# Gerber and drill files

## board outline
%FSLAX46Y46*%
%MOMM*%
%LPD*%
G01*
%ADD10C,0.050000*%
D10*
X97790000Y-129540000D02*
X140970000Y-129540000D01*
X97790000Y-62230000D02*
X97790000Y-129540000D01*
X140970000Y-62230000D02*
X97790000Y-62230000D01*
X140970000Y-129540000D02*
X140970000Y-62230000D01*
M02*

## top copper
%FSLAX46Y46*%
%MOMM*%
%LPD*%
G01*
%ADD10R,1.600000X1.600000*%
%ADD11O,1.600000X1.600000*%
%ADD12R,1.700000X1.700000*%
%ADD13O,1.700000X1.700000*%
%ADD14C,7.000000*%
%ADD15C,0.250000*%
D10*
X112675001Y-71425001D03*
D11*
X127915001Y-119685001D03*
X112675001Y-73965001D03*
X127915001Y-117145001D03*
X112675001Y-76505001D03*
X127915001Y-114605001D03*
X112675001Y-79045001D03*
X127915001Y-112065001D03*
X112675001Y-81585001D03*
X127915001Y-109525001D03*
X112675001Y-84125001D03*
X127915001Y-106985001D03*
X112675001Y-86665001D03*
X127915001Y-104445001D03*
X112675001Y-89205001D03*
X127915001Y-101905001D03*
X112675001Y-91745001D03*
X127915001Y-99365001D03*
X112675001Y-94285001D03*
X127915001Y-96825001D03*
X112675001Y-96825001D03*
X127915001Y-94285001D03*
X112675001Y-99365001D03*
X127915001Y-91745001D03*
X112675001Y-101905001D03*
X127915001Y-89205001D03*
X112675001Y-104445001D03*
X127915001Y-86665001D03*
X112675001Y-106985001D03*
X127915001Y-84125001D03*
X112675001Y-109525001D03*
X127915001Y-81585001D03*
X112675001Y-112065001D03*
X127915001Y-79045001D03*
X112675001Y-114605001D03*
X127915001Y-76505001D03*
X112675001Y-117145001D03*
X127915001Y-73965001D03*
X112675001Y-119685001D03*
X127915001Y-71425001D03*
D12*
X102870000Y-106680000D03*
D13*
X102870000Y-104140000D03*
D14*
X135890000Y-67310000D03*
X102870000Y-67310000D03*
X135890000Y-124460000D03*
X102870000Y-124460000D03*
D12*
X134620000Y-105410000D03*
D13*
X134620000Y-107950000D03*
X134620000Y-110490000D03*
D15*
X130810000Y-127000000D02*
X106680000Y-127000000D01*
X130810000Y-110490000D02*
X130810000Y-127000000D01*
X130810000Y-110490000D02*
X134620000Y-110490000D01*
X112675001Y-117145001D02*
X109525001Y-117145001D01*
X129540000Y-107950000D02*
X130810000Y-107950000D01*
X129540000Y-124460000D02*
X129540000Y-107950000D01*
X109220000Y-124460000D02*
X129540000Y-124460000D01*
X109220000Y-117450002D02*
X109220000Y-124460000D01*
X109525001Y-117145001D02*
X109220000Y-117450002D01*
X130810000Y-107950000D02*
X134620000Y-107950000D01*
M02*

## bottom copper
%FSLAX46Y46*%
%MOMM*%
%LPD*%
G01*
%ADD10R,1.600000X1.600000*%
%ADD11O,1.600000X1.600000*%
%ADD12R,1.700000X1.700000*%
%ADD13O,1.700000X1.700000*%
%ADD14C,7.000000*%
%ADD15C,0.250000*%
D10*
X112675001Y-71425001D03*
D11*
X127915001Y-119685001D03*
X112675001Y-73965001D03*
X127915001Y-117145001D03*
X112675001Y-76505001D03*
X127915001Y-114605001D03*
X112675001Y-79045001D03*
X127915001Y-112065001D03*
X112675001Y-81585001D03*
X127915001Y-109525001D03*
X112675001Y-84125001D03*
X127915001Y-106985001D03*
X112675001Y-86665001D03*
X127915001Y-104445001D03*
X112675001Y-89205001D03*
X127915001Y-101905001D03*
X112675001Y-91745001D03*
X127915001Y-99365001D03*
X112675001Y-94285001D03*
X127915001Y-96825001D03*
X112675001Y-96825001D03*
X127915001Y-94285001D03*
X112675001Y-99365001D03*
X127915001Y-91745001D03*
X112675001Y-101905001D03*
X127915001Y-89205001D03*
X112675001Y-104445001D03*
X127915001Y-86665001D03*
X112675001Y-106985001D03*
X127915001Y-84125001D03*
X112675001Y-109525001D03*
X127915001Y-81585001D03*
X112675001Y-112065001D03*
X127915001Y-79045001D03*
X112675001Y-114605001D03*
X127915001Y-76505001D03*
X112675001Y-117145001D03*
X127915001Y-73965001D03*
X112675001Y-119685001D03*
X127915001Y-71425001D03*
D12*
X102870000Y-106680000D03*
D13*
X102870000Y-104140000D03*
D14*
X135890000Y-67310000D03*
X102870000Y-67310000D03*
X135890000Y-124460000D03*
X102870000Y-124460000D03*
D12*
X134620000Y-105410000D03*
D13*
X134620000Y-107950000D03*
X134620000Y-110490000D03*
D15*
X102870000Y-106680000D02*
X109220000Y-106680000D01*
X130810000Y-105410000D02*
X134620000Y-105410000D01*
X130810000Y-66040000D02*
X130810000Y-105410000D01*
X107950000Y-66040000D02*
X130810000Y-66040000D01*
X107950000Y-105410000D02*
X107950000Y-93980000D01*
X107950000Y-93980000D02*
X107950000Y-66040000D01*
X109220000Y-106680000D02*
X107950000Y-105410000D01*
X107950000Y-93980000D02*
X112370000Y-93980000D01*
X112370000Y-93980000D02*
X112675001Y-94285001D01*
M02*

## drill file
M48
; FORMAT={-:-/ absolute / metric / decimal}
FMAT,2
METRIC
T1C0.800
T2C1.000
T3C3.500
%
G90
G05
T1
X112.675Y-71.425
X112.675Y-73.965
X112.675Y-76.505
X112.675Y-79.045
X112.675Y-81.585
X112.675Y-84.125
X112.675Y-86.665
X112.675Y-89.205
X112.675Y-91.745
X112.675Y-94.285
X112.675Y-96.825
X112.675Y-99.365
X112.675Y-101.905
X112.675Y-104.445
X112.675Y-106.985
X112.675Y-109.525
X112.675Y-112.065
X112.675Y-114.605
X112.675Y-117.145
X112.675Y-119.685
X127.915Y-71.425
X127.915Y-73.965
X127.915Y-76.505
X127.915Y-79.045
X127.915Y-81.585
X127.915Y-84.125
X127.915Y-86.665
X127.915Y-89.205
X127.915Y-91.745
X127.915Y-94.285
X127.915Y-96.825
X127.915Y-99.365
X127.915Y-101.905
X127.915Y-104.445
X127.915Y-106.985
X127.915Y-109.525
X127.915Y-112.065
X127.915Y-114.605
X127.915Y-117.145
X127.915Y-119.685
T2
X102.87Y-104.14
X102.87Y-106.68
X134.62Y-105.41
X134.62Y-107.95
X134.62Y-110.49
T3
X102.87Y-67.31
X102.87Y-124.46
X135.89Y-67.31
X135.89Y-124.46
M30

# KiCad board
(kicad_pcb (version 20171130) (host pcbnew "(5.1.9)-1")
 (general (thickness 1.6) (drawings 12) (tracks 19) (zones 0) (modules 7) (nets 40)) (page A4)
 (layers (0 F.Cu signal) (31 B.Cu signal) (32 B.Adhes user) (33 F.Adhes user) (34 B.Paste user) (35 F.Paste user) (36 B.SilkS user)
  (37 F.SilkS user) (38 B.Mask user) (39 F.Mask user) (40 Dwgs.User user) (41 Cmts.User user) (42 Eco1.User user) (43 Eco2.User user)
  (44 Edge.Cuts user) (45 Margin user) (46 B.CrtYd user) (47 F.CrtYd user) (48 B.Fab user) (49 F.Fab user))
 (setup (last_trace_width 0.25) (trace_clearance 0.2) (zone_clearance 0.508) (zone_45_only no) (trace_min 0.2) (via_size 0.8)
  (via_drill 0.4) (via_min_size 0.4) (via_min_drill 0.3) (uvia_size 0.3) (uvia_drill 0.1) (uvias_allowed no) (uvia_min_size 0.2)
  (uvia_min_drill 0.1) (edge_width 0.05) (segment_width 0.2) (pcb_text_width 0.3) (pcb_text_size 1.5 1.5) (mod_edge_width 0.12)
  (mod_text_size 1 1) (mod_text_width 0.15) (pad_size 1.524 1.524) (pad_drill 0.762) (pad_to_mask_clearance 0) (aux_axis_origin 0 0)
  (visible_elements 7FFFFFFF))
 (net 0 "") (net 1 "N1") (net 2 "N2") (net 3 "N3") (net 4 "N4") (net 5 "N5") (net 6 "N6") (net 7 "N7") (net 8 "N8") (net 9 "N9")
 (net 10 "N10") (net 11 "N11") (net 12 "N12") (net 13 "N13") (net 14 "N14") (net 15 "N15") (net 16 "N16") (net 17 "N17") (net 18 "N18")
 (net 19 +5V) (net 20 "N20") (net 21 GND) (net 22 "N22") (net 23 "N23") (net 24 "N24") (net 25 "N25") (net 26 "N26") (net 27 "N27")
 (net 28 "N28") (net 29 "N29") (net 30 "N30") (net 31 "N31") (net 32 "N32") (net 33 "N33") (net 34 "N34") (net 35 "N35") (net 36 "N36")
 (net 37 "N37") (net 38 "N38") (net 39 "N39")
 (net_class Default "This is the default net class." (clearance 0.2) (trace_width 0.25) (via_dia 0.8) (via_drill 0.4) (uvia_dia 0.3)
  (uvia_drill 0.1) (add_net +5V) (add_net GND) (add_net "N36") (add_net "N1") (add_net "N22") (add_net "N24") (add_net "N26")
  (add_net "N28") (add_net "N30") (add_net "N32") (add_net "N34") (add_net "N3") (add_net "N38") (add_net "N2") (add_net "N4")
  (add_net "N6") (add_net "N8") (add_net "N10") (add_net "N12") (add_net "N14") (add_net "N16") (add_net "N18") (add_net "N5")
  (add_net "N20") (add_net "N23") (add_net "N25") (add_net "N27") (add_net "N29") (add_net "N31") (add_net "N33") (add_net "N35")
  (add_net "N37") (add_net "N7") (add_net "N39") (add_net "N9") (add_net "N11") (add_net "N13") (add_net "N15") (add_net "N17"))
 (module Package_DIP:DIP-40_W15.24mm (layer F.Cu) (at 112.675001 71.425001)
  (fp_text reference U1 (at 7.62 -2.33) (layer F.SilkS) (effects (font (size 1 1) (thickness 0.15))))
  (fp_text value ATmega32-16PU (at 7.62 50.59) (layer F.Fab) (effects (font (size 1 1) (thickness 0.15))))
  (pad 1 thru_hole rect (at 0 0) (size 1.6 1.6) (drill 0.8) (layers *.Cu *.Mask) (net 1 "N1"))
  (pad 21 thru_hole oval (at 15.24 48.26) (size 1.6 1.6) (drill 0.8) (layers *.Cu *.Mask) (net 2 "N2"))
  (pad 2 thru_hole oval (at 0 2.54) (size 1.6 1.6) (drill 0.8) (layers *.Cu *.Mask) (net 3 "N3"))
  (pad 22 thru_hole oval (at 15.24 45.72) (size 1.6 1.6) (drill 0.8) (layers *.Cu *.Mask) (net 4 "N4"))
  (pad 3 thru_hole oval (at 0 5.08) (size 1.6 1.6) (drill 0.8) (layers *.Cu *.Mask) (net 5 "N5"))
  (pad 23 thru_hole oval (at 15.24 43.18) (size 1.6 1.6) (drill 0.8) (layers *.Cu *.Mask) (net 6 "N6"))
  (pad 4 thru_hole oval (at 0 7.62) (size 1.6 1.6) (drill 0.8) (layers *.Cu *.Mask) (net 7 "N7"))
  (pad 24 thru_hole oval (at 15.24 40.64) (size 1.6 1.6) (drill 0.8) (layers *.Cu *.Mask) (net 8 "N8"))
  (pad 5 thru_hole oval (at 0 10.16) (size 1.6 1.6) (drill 0.8) (layers *.Cu *.Mask) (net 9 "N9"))
  (pad 25 thru_hole oval (at 15.24 38.1) (size 1.6 1.6) (drill 0.8) (layers *.Cu *.Mask) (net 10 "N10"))
  (pad 6 thru_hole oval (at 0 12.7) (size 1.6 1.6) (drill 0.8) (layers *.Cu *.Mask) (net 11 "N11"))
  (pad 26 thru_hole oval (at 15.24 35.56) (size 1.6 1.6) (drill 0.8) (layers *.Cu *.Mask) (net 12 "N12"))
  (pad 7 thru_hole oval (at 0 15.24) (size 1.6 1.6) (drill 0.8) (layers *.Cu *.Mask) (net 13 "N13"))
  (pad 27 thru_hole oval (at 15.24 33.02) (size 1.6 1.6) (drill 0.8) (layers *.Cu *.Mask) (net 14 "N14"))
  (pad 8 thru_hole oval (at 0 17.78) (size 1.6 1.6) (drill 0.8) (layers *.Cu *.Mask) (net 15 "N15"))
  (pad 28 thru_hole oval (at 15.24 30.48) (size 1.6 1.6) (drill 0.8) (layers *.Cu *.Mask) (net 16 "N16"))
  (pad 9 thru_hole oval (at 0 20.32) (size 1.6 1.6) (drill 0.8) (layers *.Cu *.Mask) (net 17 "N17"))
  (pad 29 thru_hole oval (at 15.24 27.94) (size 1.6 1.6) (drill 0.8) (layers *.Cu *.Mask) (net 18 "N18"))
  (pad 10 thru_hole oval (at 0 22.86) (size 1.6 1.6) (drill 0.8) (layers *.Cu *.Mask) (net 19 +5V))
  (pad 30 thru_hole oval (at 15.24 25.4) (size 1.6 1.6) (drill 0.8) (layers *.Cu *.Mask) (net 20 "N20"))
  (pad 11 thru_hole oval (at 0 25.4) (size 1.6 1.6) (drill 0.8) (layers *.Cu *.Mask) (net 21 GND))
  (pad 31 thru_hole oval (at 15.24 22.86) (size 1.6 1.6) (drill 0.8) (layers *.Cu *.Mask) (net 21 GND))
  (pad 12 thru_hole oval (at 0 27.94) (size 1.6 1.6) (drill 0.8) (layers *.Cu *.Mask) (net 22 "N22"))
  (pad 32 thru_hole oval (at 15.24 20.32) (size 1.6 1.6) (drill 0.8) (layers *.Cu *.Mask) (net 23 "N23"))
  (pad 13 thru_hole oval (at 0 30.48) (size 1.6 1.6) (drill 0.8) (layers *.Cu *.Mask) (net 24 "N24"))
  (pad 33 thru_hole oval (at 15.24 17.78) (size 1.6 1.6) (drill 0.8) (layers *.Cu *.Mask) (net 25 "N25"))
  (pad 14 thru_hole oval (at 0 33.02) (size 1.6 1.6) (drill 0.8) (layers *.Cu *.Mask) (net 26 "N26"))
  (pad 34 thru_hole oval (at 15.24 15.24) (size 1.6 1.6) (drill 0.8) (layers *.Cu *.Mask) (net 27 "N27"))
  (pad 15 thru_hole oval (at 0 35.56) (size 1.6 1.6) (drill 0.8) (layers *.Cu *.Mask) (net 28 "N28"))
  (pad 35 thru_hole oval (at 15.24 12.7) (size 1.6 1.6) (drill 0.8) (layers *.Cu *.Mask) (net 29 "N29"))
  (pad 16 thru_hole oval (at 0 38.1) (size 1.6 1.6) (drill 0.8) (layers *.Cu *.Mask) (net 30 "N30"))
  (pad 36 thru_hole oval (at 15.24 10.16) (size 1.6 1.6) (drill 0.8) (layers *.Cu *.Mask) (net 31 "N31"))
  (pad 17 thru_hole oval (at 0 40.64) (size 1.6 1.6) (drill 0.8) (layers *.Cu *.Mask) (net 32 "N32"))
  (pad 37 thru_hole oval (at 15.24 7.62) (size 1.6 1.6) (drill 0.8) (layers *.Cu *.Mask) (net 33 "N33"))
  (pad 18 thru_hole oval (at 0 43.18) (size 1.6 1.6) (drill 0.8) (layers *.Cu *.Mask) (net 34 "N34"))
  (pad 38 thru_hole oval (at 15.24 5.08) (size 1.6 1.6) (drill 0.8) (layers *.Cu *.Mask) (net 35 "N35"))
  (pad 19 thru_hole oval (at 0 45.72) (size 1.6 1.6) (drill 0.8) (layers *.Cu *.Mask) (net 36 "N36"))
  (pad 39 thru_hole oval (at 15.24 2.54) (size 1.6 1.6) (drill 0.8) (layers *.Cu *.Mask) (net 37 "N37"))
  (pad 20 thru_hole oval (at 0 48.26) (size 1.6 1.6) (drill 0.8) (layers *.Cu *.Mask) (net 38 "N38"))
  (pad 40 thru_hole oval (at 15.24 0) (size 1.6 1.6) (drill 0.8) (layers *.Cu *.Mask) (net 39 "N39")))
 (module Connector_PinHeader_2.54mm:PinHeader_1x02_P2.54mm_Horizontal (layer F.Cu) (at 102.87 106.68 180)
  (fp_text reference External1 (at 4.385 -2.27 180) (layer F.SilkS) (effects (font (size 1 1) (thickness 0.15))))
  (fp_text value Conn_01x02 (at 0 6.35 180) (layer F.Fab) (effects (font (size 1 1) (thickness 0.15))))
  (pad 1 thru_hole rect (at 0 0 180) (size 1.7 1.7) (drill 1) (layers *.Cu *.Mask) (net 19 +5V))
  (pad 2 thru_hole oval (at 0 2.54 180) (size 1.7 1.7) (drill 1) (layers *.Cu *.Mask) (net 21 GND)))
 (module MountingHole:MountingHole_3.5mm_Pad (layer F.Cu) (at 135.89 67.31)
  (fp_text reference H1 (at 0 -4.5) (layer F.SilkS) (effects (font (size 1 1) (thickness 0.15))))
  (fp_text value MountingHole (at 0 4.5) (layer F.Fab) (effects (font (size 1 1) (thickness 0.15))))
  (pad 1 thru_hole circle (at 0 0) (size 7 7) (drill 3.5) (layers *.Cu *.Mask)))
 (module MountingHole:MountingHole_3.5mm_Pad (layer F.Cu) (at 102.87 67.31)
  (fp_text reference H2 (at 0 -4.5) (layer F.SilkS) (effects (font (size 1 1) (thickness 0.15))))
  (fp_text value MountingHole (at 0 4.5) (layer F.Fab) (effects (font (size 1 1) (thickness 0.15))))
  (pad 1 thru_hole circle (at 0 0) (size 7 7) (drill 3.5) (layers *.Cu *.Mask)))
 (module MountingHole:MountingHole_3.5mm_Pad (layer F.Cu) (at 135.89 124.46)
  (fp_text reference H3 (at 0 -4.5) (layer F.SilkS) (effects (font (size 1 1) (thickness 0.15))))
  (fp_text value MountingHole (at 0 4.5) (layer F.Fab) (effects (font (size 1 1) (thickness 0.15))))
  (pad 1 thru_hole circle (at 0 0) (size 7 7) (drill 3.5) (layers *.Cu *.Mask)))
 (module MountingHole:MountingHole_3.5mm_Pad (layer F.Cu) (at 102.87 124.46)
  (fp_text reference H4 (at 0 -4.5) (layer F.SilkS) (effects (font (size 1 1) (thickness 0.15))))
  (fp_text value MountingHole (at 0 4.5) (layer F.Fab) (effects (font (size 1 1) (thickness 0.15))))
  (pad 1 thru_hole circle (at 0 0) (size 7 7) (drill 3.5) (layers *.Cu *.Mask)))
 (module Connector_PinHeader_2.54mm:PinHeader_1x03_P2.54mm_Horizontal (layer F.Cu) (at 134.62 105.41)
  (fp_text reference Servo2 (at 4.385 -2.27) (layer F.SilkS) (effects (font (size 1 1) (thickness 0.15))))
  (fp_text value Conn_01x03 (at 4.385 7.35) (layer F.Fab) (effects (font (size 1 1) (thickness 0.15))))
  (pad 1 thru_hole rect (at 0 0) (size 1.7 1.7) (drill 1) (layers *.Cu *.Mask) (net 19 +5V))
  (pad 2 thru_hole oval (at 0 2.54) (size 1.7 1.7) (drill 1) (layers *.Cu *.Mask) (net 36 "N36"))
  (pad 3 thru_hole oval (at 0 5.08) (size 1.7 1.7) (drill 1) (layers *.Cu *.Mask) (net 21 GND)))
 (gr_line (start 97.79 129.54) (end 140.97 129.54) (angle 90) (layer Edge.Cuts) (width 0.05))
 (gr_line (start 97.79 62.23) (end 97.79 129.54) (angle 90) (layer Edge.Cuts) (width 0.05))
 (gr_line (start 140.97 62.23) (end 97.79 62.23) (angle 90) (layer Edge.Cuts) (width 0.05))
 (gr_line (start 140.97 129.54) (end 140.97 62.23) (angle 90) (layer Edge.Cuts) (width 0.05))
 (segment (start 102.87 106.68) (end 109.22 106.68) (width 0.25) (layer B.Cu) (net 19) (status 400000))
 (segment (start 130.81 105.41) (end 134.62 105.41) (width 0.25) (layer B.Cu) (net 19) (status 800000))
 (segment (start 130.81 66.04) (end 130.81 105.41) (width 0.25) (layer B.Cu) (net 19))
 (segment (start 107.95 66.04) (end 130.81 66.04) (width 0.25) (layer B.Cu) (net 19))
 (segment (start 107.95 105.41) (end 107.95 93.98) (width 0.25) (layer B.Cu) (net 19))
 (segment (start 107.95 93.98) (end 107.95 66.04) (width 0.25) (layer B.Cu) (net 19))
 (segment (start 109.22 106.68) (end 107.95 105.41) (width 0.25) (layer B.Cu) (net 19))
 (segment (start 107.95 93.98) (end 112.37 93.98) (width 0.25) (layer B.Cu) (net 19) (status 800000))
 (segment (start 112.37 93.98) (end 112.675001 94.285001) (width 0.25) (layer B.Cu) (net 19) (status C00000))
 (segment (start 130.81 127) (end 106.68 127) (width 0.25) (layer F.Cu) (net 21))
 (segment (start 130.81 110.49) (end 130.81 127) (width 0.25) (layer F.Cu) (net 21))
 (segment (start 130.81 110.49) (end 134.62 110.49) (width 0.25) (layer F.Cu) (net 21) (status 800000))
 (segment (start 112.675001 117.145001) (end 109.525001 117.145001) (width 0.25) (layer F.Cu) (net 36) (status 400000))
 (segment (start 129.54 107.95) (end 130.81 107.95) (width 0.25) (layer F.Cu) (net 36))
 (segment (start 129.54 124.46) (end 129.54 107.95) (width 0.25) (layer F.Cu) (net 36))
 (segment (start 109.22 124.46) (end 129.54 124.46) (width 0.25) (layer F.Cu) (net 36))
 (segment (start 109.22 117.450002) (end 109.22 124.46) (width 0.25) (layer F.Cu) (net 36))
 (segment (start 109.525001 117.145001) (end 109.22 117.450002) (width 0.25) (layer F.Cu) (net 36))
 (segment (start 130.81 107.95) (end 134.62 107.95) (width 0.25) (layer F.Cu) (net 36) (status 800000)))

